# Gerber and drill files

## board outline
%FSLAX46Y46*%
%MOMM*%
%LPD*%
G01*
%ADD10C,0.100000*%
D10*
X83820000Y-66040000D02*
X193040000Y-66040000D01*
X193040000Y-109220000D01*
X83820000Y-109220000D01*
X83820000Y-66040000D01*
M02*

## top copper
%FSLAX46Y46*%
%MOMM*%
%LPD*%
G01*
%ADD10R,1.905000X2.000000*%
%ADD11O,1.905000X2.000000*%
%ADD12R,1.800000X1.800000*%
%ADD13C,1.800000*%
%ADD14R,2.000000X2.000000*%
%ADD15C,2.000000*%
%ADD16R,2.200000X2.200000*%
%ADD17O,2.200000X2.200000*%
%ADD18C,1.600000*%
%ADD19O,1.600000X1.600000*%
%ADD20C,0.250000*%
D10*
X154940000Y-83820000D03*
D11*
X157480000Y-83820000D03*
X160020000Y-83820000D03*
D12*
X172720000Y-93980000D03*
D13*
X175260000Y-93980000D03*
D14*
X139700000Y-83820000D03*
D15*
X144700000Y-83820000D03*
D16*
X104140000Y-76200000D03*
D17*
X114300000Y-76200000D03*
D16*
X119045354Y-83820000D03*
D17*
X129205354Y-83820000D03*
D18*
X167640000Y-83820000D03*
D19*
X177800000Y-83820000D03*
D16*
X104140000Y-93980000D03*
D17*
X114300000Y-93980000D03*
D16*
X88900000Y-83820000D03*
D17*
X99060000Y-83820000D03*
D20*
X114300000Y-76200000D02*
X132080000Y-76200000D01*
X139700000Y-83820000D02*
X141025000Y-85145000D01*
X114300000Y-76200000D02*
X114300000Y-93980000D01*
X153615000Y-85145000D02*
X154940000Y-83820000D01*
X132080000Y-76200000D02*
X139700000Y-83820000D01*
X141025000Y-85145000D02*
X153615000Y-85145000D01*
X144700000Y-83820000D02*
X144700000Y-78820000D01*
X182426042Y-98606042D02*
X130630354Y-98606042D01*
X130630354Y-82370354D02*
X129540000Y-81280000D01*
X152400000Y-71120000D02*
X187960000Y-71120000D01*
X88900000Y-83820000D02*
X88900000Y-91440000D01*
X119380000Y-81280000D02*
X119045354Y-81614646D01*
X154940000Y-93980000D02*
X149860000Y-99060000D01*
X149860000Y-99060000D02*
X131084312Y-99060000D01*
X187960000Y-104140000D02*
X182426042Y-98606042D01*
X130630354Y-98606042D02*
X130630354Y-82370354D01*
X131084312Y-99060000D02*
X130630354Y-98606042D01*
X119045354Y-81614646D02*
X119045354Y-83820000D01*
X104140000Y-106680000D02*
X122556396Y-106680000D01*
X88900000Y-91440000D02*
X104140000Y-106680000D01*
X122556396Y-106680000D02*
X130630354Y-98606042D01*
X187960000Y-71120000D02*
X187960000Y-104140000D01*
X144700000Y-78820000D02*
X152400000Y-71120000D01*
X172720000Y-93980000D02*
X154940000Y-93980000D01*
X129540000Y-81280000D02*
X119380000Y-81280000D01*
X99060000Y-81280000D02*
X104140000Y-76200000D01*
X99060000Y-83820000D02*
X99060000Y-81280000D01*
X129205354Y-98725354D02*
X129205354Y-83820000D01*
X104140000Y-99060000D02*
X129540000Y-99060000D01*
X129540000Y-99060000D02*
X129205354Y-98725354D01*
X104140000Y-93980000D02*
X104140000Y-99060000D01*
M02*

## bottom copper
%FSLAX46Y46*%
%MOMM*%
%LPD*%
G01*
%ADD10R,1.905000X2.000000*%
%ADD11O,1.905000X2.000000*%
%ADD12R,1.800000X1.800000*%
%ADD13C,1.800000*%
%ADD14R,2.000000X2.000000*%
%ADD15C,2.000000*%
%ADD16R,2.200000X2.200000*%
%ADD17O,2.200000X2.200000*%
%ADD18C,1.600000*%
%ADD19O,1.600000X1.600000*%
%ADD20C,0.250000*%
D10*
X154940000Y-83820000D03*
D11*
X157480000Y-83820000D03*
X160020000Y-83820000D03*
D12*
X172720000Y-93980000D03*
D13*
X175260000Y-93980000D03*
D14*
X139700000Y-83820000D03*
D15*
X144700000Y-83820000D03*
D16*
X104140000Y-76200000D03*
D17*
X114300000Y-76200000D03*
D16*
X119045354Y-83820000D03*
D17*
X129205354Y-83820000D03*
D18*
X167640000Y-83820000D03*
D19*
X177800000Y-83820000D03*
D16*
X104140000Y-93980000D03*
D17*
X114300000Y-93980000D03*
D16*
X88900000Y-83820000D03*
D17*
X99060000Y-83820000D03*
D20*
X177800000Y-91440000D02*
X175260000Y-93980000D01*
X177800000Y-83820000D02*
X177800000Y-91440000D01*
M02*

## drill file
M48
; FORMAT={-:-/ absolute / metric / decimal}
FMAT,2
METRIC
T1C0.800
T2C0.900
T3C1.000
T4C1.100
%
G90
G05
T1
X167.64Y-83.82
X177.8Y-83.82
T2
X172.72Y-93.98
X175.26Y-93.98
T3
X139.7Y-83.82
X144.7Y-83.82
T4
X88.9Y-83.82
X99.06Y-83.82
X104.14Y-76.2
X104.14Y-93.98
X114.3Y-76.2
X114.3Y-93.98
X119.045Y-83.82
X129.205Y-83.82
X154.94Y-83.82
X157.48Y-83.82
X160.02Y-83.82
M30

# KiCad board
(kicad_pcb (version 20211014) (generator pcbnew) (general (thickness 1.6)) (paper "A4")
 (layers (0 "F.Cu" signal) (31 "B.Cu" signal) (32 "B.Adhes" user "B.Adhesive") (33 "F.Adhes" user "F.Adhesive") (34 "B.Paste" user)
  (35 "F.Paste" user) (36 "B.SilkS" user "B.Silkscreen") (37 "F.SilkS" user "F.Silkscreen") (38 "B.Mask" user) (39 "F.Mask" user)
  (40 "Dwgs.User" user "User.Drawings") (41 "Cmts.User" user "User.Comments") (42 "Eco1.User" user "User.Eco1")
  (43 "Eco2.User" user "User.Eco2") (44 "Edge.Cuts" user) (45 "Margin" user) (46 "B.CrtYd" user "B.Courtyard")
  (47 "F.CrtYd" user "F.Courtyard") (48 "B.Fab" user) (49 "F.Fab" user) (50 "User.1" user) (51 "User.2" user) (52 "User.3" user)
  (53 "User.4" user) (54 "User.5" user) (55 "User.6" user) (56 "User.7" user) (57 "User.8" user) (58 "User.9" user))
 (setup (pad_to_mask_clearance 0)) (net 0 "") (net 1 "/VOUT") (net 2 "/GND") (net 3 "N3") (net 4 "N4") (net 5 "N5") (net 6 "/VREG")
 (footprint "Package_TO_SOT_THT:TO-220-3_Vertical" (layer "F.Cu") (at 154.94 83.82)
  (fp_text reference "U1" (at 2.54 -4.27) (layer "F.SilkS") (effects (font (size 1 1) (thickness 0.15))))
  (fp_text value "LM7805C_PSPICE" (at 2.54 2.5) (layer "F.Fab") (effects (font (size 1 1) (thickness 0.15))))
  (pad "1" thru_hole rect (at 0 0) (size 1.905 2) (drill oval 1.1) (layers *.Cu *.Mask) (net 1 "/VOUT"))
  (pad "2" thru_hole oval (at 2.54 0) (size 1.905 2) (drill 1.1) (layers *.Cu *.Mask))
  (pad "3" thru_hole oval (at 5.08 0) (size 1.905 2) (drill 1.1) (layers *.Cu *.Mask)))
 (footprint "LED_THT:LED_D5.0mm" (layer "F.Cu") (at 172.72 93.98)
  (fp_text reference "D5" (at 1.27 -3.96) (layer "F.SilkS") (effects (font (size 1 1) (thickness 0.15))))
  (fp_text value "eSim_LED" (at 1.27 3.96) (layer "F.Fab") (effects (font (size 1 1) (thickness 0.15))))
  (pad "1" thru_hole rect (at 0 0) (size 1.8 1.8) (drill 0.9) (layers *.Cu *.Mask) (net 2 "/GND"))
  (pad "2" thru_hole circle (at 2.54 0) (size 1.8 1.8) (drill 0.9) (layers *.Cu *.Mask) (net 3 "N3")))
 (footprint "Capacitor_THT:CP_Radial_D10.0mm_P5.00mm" (layer "F.Cu") (at 139.7 83.82)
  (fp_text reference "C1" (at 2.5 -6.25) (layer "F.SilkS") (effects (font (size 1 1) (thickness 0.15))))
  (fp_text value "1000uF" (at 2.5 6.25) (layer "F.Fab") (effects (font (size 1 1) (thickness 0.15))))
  (pad "1" thru_hole rect (at 0 0) (size 2 2) (drill 1) (layers *.Cu *.Mask) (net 1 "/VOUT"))
  (pad "2" thru_hole circle (at 5 0) (size 2 2) (drill 1) (layers *.Cu *.Mask) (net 2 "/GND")))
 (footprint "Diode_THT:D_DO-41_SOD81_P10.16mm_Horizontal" (layer "F.Cu") (at 104.14 76.2)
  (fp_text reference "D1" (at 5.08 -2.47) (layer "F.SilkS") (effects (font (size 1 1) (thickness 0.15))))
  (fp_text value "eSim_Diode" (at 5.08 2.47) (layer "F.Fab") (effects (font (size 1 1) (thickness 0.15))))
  (pad "1" thru_hole rect (at 0 0) (size 2.2 2.2) (drill 1.1) (layers *.Cu *.Mask) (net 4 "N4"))
  (pad "2" thru_hole oval (at 10.16 0) (size 2.2 2.2) (drill 1.1) (layers *.Cu *.Mask) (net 1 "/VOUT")))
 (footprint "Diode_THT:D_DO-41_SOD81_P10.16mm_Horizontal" (layer "F.Cu") (at 119.045354 83.82)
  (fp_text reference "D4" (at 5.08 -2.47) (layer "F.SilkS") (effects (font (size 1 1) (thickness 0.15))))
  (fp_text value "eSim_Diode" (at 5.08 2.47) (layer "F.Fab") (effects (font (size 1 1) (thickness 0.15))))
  (pad "1" thru_hole rect (at 0 0) (size 2.2 2.2) (drill 1.1) (layers *.Cu *.Mask) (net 2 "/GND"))
  (pad "2" thru_hole oval (at 10.16 0) (size 2.2 2.2) (drill 1.1) (layers *.Cu *.Mask) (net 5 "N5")))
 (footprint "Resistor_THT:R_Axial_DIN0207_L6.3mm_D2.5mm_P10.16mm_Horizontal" (layer "F.Cu") (at 167.64 83.82)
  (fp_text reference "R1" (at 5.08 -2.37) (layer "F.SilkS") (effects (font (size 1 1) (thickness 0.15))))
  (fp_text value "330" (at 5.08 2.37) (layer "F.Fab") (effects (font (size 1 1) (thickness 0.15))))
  (pad "1" thru_hole circle (at 0 0) (size 1.6 1.6) (drill 0.8) (layers *.Cu *.Mask) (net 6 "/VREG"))
  (pad "2" thru_hole oval (at 10.16 0) (size 1.6 1.6) (drill 0.8) (layers *.Cu *.Mask) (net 3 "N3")))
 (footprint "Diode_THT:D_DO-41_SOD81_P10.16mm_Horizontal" (layer "F.Cu") (at 104.14 93.98)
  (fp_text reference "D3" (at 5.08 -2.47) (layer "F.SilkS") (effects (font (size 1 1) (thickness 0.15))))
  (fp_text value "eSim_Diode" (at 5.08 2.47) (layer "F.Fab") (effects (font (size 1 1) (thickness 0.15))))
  (pad "1" thru_hole rect (at 0 0) (size 2.2 2.2) (drill 1.1) (layers *.Cu *.Mask) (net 5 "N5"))
  (pad "2" thru_hole oval (at 10.16 0) (size 2.2 2.2) (drill 1.1) (layers *.Cu *.Mask) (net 1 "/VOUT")))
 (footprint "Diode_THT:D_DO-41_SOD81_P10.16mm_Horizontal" (layer "F.Cu") (at 88.9 83.82)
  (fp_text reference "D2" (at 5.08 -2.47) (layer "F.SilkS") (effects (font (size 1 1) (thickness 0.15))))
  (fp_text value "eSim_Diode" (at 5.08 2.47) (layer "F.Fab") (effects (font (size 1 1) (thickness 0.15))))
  (pad "1" thru_hole rect (at 0 0) (size 2.2 2.2) (drill 1.1) (layers *.Cu *.Mask) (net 2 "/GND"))
  (pad "2" thru_hole oval (at 10.16 0) (size 2.2 2.2) (drill 1.1) (layers *.Cu *.Mask) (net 4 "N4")))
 (gr_rect (start 83.82 66.04) (end 193.04 109.22) (layer "Edge.Cuts") (width 0.1) (fill none))
 (segment (start 114.3 76.2) (end 132.08 76.2) (width 0.25) (layer "F.Cu") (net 1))
 (segment (start 139.7 83.82) (end 141.025 85.145) (width 0.25) (layer "F.Cu") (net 1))
 (segment (start 114.3 76.2) (end 114.3 93.98) (width 0.25) (layer "F.Cu") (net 1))
 (segment (start 153.615 85.145) (end 154.94 83.82) (width 0.25) (layer "F.Cu") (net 1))
 (segment (start 132.08 76.2) (end 139.7 83.82) (width 0.25) (layer "F.Cu") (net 1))
 (segment (start 141.025 85.145) (end 153.615 85.145) (width 0.25) (layer "F.Cu") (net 1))
 (segment (start 144.7 83.82) (end 144.7 78.82) (width 0.25) (layer "F.Cu") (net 2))
 (segment (start 182.426042 98.606042) (end 130.630354 98.606042) (width 0.25) (layer "F.Cu") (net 2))
 (segment (start 130.630354 82.370354) (end 129.54 81.28) (width 0.25) (layer "F.Cu") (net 2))
 (segment (start 152.4 71.12) (end 187.96 71.12) (width 0.25) (layer "F.Cu") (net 2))
 (segment (start 88.9 83.82) (end 88.9 91.44) (width 0.25) (layer "F.Cu") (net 2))
 (segment (start 119.38 81.28) (end 119.045354 81.614646) (width 0.25) (layer "F.Cu") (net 2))
 (segment (start 154.94 93.98) (end 149.86 99.06) (width 0.25) (layer "F.Cu") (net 2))
 (segment (start 149.86 99.06) (end 131.084312 99.06) (width 0.25) (layer "F.Cu") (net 2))
 (segment (start 187.96 104.14) (end 182.426042 98.606042) (width 0.25) (layer "F.Cu") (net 2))
 (segment (start 130.630354 98.606042) (end 130.630354 82.370354) (width 0.25) (layer "F.Cu") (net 2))
 (segment (start 131.084312 99.06) (end 130.630354 98.606042) (width 0.25) (layer "F.Cu") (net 2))
 (segment (start 119.045354 81.614646) (end 119.045354 83.82) (width 0.25) (layer "F.Cu") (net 2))
 (segment (start 104.14 106.68) (end 122.556396 106.68) (width 0.25) (layer "F.Cu") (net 2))
 (segment (start 88.9 91.44) (end 104.14 106.68) (width 0.25) (layer "F.Cu") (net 2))
 (segment (start 122.556396 106.68) (end 130.630354 98.606042) (width 0.25) (layer "F.Cu") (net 2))
 (segment (start 187.96 71.12) (end 187.96 104.14) (width 0.25) (layer "F.Cu") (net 2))
 (segment (start 144.7 78.82) (end 152.4 71.12) (width 0.25) (layer "F.Cu") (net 2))
 (segment (start 172.72 93.98) (end 154.94 93.98) (width 0.25) (layer "F.Cu") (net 2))
 (segment (start 129.54 81.28) (end 119.38 81.28) (width 0.25) (layer "F.Cu") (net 2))
 (segment (start 99.06 81.28) (end 104.14 76.2) (width 0.25) (layer "F.Cu") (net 4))
 (segment (start 99.06 83.82) (end 99.06 81.28) (width 0.25) (layer "F.Cu") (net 4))
 (segment (start 129.205354 98.725354) (end 129.205354 83.82) (width 0.25) (layer "F.Cu") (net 5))
 (segment (start 104.14 99.06) (end 129.54 99.06) (width 0.25) (layer "F.Cu") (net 5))
 (segment (start 129.54 99.06) (end 129.205354 98.725354) (width 0.25) (layer "F.Cu") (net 5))
 (segment (start 104.14 93.98) (end 104.14 99.06) (width 0.25) (layer "F.Cu") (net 5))
 (segment (start 177.8 91.44) (end 175.26 93.98) (width 0.25) (layer "B.Cu") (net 3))
 (segment (start 177.8 83.82) (end 177.8 91.44) (width 0.25) (layer "B.Cu") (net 3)))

